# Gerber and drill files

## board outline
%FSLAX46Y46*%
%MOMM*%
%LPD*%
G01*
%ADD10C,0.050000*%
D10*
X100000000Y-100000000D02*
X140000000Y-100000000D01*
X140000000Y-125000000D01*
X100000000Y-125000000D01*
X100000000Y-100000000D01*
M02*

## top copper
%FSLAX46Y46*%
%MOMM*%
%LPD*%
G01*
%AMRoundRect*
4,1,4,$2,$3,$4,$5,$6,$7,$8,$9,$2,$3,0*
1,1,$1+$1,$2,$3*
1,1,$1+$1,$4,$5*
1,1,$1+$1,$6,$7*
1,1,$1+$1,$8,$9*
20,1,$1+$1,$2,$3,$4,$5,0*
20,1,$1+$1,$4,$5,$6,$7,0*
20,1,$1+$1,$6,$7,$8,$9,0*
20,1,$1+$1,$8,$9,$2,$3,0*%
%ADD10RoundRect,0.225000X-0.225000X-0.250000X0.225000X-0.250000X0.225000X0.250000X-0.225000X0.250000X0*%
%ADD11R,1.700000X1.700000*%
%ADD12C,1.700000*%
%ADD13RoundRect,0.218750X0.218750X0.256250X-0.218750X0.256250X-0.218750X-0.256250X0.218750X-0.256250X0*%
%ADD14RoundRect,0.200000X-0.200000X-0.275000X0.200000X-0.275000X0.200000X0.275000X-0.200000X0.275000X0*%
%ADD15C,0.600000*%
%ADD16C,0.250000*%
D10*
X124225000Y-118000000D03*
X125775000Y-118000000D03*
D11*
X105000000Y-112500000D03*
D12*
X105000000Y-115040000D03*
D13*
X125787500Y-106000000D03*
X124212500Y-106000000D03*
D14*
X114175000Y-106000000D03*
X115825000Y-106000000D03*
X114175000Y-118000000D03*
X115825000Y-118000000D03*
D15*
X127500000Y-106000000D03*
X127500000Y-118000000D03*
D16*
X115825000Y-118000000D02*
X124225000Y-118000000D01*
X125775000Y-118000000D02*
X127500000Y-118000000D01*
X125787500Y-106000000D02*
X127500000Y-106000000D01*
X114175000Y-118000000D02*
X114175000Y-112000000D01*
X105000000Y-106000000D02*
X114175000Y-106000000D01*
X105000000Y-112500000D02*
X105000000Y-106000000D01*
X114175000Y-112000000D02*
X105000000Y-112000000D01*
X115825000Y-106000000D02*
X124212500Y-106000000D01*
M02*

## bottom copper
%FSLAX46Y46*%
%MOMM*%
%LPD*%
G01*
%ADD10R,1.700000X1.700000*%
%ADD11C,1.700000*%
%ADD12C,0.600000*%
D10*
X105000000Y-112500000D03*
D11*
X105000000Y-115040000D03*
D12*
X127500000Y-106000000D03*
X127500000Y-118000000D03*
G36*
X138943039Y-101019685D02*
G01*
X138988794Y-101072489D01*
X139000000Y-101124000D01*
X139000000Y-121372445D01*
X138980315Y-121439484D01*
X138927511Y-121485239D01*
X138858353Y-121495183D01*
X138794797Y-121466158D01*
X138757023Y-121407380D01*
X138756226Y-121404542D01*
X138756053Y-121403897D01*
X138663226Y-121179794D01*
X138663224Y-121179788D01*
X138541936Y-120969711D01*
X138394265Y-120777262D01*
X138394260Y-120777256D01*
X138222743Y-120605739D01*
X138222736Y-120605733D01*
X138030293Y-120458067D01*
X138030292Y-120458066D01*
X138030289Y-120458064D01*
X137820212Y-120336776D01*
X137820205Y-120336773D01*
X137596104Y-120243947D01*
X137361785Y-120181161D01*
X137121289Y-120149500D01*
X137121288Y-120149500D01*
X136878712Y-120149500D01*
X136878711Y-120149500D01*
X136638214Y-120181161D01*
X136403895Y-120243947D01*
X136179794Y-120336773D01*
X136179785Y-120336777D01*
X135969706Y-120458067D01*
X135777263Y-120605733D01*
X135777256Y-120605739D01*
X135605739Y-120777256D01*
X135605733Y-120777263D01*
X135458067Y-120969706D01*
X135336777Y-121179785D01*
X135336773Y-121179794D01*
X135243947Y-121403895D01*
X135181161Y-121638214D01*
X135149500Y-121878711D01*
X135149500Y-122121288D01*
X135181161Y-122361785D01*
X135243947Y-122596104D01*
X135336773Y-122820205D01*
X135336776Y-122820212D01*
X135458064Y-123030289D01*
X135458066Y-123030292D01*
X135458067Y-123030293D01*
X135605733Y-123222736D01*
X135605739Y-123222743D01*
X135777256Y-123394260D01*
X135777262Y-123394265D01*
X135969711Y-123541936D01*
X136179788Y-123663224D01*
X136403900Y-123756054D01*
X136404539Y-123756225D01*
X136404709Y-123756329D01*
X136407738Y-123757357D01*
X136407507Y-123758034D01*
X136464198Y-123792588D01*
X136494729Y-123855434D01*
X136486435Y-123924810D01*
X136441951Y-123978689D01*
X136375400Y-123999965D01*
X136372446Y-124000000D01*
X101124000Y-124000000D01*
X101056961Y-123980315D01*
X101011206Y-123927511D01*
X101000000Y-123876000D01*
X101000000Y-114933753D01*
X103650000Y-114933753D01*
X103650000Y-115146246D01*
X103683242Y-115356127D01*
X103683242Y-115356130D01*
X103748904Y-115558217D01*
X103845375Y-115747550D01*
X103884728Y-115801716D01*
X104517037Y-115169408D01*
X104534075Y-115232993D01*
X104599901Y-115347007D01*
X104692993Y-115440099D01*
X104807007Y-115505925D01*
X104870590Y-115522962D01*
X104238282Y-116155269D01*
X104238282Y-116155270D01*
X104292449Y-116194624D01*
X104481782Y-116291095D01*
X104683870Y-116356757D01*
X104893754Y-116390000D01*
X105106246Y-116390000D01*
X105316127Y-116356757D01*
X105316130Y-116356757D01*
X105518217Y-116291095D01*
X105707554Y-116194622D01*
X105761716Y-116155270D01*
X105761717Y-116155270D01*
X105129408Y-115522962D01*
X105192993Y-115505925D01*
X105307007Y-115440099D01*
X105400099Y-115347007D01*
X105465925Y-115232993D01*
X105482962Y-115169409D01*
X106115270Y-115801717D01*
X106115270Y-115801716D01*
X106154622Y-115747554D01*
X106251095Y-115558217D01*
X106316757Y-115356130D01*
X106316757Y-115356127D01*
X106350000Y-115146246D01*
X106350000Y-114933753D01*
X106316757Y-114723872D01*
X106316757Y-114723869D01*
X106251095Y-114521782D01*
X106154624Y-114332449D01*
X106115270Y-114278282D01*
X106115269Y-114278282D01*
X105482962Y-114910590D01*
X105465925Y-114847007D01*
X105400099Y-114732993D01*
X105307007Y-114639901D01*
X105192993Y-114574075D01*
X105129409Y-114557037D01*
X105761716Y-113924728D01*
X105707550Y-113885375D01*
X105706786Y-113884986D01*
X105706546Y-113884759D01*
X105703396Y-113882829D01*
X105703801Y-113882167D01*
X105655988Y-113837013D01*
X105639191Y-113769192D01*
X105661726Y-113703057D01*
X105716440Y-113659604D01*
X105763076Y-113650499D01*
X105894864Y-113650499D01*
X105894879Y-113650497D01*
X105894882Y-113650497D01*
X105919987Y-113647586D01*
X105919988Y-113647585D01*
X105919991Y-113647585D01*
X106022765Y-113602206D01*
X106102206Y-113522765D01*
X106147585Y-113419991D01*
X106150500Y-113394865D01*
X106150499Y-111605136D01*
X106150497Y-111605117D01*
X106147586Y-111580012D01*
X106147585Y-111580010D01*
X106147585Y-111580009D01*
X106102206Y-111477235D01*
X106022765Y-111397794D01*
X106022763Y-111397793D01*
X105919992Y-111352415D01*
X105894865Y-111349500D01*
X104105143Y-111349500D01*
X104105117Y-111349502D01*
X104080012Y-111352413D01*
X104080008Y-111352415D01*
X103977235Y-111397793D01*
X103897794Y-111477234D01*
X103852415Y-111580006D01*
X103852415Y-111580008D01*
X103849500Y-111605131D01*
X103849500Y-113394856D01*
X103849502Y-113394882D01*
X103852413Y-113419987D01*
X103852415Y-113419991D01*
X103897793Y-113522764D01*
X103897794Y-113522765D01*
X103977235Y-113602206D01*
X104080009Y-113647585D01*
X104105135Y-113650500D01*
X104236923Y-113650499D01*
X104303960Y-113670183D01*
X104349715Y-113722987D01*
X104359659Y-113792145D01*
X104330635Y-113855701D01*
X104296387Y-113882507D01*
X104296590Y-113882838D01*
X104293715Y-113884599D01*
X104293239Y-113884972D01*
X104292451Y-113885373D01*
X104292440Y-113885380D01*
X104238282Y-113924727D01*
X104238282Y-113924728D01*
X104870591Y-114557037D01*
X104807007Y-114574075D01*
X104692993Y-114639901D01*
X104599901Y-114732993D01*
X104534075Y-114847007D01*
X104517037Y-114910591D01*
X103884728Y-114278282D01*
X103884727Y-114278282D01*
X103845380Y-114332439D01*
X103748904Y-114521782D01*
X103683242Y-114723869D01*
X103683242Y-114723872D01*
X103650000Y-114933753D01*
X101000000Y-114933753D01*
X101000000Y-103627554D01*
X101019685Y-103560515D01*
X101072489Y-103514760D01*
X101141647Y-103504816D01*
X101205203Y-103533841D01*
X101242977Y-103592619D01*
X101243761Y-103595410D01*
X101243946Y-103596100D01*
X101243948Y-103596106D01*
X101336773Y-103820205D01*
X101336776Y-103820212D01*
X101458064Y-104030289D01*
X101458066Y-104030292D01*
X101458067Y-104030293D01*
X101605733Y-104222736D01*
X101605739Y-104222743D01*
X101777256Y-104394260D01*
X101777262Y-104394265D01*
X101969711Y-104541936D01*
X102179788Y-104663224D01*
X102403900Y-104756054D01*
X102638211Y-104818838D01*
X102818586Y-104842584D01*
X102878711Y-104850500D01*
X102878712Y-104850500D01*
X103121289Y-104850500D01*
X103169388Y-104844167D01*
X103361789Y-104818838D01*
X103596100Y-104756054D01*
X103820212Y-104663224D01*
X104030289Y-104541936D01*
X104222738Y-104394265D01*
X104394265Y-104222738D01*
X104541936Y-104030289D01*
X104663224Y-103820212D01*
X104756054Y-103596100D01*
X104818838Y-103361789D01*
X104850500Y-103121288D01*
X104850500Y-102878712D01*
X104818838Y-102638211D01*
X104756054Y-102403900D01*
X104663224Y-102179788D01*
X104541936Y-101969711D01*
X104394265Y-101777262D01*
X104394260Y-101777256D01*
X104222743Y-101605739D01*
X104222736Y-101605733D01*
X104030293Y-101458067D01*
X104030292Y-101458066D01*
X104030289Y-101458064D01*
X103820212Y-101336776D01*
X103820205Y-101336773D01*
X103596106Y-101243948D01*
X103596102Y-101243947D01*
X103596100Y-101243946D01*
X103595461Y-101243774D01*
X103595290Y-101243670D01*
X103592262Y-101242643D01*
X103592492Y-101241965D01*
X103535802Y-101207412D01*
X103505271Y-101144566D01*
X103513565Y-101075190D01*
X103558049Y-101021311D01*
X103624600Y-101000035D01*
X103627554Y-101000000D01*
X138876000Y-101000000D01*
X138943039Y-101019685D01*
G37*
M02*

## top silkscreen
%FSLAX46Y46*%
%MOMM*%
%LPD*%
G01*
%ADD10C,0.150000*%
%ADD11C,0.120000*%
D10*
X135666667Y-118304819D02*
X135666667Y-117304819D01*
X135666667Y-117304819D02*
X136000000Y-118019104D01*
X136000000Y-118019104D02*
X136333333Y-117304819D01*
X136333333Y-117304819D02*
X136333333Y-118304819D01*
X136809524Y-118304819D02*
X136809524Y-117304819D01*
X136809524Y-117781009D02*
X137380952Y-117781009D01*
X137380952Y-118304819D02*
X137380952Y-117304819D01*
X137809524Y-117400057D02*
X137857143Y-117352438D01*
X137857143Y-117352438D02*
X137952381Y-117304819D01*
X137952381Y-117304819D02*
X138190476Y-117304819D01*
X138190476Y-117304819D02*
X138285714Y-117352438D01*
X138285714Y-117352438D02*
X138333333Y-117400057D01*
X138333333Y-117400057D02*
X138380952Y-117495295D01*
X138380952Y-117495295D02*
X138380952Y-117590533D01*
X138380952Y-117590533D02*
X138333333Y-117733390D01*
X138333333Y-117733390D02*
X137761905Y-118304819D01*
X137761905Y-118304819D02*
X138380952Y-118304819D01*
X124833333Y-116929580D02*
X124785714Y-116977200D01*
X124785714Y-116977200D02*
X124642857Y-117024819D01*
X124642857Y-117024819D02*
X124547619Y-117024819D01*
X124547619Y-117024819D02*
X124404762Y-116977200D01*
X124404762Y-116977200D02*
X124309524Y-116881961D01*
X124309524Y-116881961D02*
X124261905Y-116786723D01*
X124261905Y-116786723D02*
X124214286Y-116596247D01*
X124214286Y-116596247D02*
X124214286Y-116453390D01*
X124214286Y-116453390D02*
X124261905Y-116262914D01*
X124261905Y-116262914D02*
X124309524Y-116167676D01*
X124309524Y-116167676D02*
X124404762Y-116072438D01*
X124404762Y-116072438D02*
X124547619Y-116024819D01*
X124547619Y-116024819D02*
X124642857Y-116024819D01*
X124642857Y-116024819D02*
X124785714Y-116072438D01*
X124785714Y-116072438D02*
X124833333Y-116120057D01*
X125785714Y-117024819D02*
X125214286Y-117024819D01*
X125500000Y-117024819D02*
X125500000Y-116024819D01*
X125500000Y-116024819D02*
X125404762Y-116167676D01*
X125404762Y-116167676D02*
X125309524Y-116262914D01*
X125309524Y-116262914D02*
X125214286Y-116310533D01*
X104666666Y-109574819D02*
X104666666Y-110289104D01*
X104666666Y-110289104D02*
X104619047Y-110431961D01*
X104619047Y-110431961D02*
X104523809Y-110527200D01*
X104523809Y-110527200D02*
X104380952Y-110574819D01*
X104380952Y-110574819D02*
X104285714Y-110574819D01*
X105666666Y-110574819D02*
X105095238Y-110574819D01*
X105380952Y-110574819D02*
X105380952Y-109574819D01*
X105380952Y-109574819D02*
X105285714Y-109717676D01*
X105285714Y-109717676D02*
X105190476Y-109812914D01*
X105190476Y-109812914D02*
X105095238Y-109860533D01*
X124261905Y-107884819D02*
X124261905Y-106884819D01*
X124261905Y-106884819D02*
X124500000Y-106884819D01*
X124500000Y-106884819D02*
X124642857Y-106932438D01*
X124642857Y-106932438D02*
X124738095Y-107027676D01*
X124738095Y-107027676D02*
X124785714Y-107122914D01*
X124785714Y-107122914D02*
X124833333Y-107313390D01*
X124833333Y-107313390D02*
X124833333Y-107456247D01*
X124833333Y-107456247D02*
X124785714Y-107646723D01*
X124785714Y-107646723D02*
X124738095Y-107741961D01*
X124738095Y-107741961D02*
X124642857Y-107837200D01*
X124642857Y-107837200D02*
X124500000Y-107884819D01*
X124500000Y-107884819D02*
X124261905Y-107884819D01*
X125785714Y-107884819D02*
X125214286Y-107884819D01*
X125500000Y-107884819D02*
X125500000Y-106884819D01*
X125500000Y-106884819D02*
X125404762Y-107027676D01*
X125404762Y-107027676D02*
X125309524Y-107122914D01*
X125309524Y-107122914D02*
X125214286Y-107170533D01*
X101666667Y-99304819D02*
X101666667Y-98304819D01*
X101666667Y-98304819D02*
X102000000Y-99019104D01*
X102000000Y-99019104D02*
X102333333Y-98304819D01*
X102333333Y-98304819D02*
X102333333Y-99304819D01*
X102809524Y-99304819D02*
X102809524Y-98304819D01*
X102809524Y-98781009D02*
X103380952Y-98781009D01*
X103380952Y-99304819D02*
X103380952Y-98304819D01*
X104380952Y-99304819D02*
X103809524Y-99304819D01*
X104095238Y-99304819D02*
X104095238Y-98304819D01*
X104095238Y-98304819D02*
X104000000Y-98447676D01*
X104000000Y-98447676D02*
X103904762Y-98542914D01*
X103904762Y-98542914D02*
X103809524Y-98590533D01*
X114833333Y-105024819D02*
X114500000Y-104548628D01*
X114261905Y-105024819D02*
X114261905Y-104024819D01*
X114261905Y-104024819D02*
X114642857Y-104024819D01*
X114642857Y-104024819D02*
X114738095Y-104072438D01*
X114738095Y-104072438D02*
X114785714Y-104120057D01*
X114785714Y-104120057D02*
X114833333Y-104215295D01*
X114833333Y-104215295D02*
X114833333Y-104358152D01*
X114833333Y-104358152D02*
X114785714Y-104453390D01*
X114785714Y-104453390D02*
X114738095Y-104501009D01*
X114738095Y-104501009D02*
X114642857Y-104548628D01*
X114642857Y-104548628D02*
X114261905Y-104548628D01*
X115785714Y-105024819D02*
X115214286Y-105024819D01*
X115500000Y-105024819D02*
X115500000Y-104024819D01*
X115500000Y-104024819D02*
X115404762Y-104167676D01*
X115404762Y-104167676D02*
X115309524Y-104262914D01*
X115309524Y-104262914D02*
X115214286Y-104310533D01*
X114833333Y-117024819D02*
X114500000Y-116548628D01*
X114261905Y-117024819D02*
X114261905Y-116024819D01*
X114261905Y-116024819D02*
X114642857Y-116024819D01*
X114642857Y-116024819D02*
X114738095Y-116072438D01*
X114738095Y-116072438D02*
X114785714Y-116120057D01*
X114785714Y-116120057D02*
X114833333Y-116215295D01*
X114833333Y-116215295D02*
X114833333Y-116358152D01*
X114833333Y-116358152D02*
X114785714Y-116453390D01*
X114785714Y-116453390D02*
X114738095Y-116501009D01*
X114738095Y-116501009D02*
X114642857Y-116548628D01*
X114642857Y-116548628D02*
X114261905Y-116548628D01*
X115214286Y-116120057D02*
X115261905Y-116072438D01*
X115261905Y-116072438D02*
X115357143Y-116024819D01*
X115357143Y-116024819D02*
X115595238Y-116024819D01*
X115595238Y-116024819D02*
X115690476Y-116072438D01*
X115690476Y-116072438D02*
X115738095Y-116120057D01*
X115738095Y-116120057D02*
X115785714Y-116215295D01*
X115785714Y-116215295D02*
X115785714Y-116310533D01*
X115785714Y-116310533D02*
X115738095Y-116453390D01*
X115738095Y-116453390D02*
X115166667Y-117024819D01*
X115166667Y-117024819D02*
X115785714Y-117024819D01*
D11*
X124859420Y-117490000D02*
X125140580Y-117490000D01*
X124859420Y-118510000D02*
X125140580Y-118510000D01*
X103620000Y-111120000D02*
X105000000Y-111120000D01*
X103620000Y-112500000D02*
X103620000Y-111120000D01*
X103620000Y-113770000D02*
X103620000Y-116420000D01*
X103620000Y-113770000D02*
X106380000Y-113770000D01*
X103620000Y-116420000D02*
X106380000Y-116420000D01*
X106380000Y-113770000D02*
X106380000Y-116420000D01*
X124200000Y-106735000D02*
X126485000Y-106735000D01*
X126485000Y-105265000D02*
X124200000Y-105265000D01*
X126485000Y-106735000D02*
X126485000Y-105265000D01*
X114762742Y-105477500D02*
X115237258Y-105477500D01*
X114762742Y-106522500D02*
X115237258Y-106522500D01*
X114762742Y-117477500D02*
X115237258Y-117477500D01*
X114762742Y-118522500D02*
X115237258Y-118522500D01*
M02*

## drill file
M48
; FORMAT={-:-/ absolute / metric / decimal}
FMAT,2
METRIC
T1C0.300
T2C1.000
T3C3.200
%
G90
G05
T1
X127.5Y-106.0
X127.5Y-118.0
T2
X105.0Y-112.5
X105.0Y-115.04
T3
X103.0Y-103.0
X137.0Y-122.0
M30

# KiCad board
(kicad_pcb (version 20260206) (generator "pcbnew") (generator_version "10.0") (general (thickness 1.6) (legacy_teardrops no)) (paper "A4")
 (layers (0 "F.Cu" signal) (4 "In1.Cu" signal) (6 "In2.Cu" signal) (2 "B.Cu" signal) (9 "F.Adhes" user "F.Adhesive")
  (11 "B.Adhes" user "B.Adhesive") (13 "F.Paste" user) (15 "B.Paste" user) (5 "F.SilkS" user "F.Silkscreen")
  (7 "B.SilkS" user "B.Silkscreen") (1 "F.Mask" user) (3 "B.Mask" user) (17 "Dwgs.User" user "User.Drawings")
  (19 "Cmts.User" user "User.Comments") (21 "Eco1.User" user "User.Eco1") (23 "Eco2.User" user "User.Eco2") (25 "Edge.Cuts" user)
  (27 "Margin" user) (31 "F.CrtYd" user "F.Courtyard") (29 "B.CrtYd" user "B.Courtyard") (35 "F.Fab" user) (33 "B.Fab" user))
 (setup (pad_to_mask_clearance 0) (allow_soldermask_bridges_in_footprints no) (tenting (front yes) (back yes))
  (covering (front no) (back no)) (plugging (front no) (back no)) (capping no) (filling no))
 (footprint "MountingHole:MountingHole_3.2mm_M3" (layer "F.Cu") (at 137 122)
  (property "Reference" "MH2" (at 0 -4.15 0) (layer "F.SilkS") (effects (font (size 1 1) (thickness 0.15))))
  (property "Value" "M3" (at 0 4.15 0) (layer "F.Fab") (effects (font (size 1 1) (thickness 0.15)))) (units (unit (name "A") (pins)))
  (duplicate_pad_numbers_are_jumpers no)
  (pad "" np_thru_hole circle (at 0 0) (size 3.2 3.2) (drill 3.2) (layers "*.Cu" "*.Mask")))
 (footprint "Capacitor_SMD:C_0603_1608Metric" (layer "F.Cu") (at 125 118)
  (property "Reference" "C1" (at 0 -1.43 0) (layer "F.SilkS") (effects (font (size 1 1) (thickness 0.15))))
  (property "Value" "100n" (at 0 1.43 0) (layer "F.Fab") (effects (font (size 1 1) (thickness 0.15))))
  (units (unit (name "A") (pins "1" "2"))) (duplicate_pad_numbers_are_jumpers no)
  (fp_line (start -0.14058 -0.51) (end 0.14058 -0.51) (stroke (width 0.12) (type solid)) (layer "F.SilkS"))
  (fp_line (start -0.14058 0.51) (end 0.14058 0.51) (stroke (width 0.12) (type solid)) (layer "F.SilkS"))
  (pad "1" smd roundrect (at -0.775 0) (size 0.9 0.95) (layers "F.Cu" "F.Mask" "F.Paste") (roundrect_rratio 0.25) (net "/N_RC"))
  (pad "2" smd roundrect (at 0.775 0) (size 0.9 0.95) (layers "F.Cu" "F.Mask" "F.Paste") (roundrect_rratio 0.25) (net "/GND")))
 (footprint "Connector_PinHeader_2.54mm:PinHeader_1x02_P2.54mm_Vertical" (layer "F.Cu") (at 105 112.5)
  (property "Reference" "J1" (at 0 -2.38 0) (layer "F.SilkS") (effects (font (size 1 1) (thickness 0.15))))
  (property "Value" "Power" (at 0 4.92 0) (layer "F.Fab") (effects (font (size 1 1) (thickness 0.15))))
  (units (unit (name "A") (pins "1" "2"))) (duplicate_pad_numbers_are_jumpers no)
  (fp_line (start -1.38 -1.38) (end 0 -1.38) (stroke (width 0.12) (type solid)) (layer "F.SilkS"))
  (fp_line (start -1.38 0) (end -1.38 -1.38) (stroke (width 0.12) (type solid)) (layer "F.SilkS"))
  (fp_line (start -1.38 1.27) (end -1.38 3.92) (stroke (width 0.12) (type solid)) (layer "F.SilkS"))
  (fp_line (start -1.38 1.27) (end 1.38 1.27) (stroke (width 0.12) (type solid)) (layer "F.SilkS"))
  (fp_line (start -1.38 3.92) (end 1.38 3.92) (stroke (width 0.12) (type solid)) (layer "F.SilkS"))
  (fp_line (start 1.38 1.27) (end 1.38 3.92) (stroke (width 0.12) (type solid)) (layer "F.SilkS"))
  (pad "1" thru_hole rect (at 0 0) (size 1.7 1.7) (drill 1) (layers "*.Cu" "*.Mask") (remove_unused_layers no) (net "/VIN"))
  (pad "2" thru_hole circle (at 0 2.54) (size 1.7 1.7) (drill 1) (layers "*.Cu" "*.Mask") (remove_unused_layers no) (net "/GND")))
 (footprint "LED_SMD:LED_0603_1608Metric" (layer "F.Cu") (at 125 106 180)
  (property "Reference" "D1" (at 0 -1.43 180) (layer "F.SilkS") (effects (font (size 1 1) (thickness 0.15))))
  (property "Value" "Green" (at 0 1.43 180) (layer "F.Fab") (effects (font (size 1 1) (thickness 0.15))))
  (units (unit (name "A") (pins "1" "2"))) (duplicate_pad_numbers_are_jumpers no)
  (fp_line (start 0.8 -0.735) (end -1.485 -0.735) (stroke (width 0.12) (type solid)) (layer "F.SilkS"))
  (fp_line (start -1.485 0.735) (end 0.8 0.735) (stroke (width 0.12) (type solid)) (layer "F.SilkS"))
  (fp_line (start -1.485 -0.735) (end -1.485 0.735) (stroke (width 0.12) (type solid)) (layer "F.SilkS"))
  (pad "1" smd roundrect (at -0.7875 0 180) (size 0.875 0.95) (layers "F.Cu" "F.Mask" "F.Paste") (roundrect_rratio 0.25) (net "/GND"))
  (pad "2" smd roundrect (at 0.7875 0 180) (size 0.875 0.95) (layers "F.Cu" "F.Mask" "F.Paste") (roundrect_rratio 0.25) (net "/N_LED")))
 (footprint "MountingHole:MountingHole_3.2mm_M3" (layer "F.Cu") (at 103 103)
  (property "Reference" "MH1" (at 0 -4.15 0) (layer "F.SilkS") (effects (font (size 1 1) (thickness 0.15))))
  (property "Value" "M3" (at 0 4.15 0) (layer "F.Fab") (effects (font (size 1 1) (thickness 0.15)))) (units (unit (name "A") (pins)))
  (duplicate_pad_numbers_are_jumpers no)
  (pad "" np_thru_hole circle (at 0 0) (size 3.2 3.2) (drill 3.2) (layers "*.Cu" "*.Mask")))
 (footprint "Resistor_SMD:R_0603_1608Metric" (layer "F.Cu") (at 115 106)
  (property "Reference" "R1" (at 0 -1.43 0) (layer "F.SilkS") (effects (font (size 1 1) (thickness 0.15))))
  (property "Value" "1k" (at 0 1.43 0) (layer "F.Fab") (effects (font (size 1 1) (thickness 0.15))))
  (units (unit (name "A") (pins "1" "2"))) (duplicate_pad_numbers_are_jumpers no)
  (fp_line (start -0.237258 -0.5225) (end 0.237258 -0.5225) (stroke (width 0.12) (type solid)) (layer "F.SilkS"))
  (fp_line (start -0.237258 0.5225) (end 0.237258 0.5225) (stroke (width 0.12) (type solid)) (layer "F.SilkS"))
  (pad "1" smd roundrect (at -0.825 0) (size 0.8 0.95) (layers "F.Cu" "F.Mask" "F.Paste") (roundrect_rratio 0.25) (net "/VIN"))
  (pad "2" smd roundrect (at 0.825 0) (size 0.8 0.95) (layers "F.Cu" "F.Mask" "F.Paste") (roundrect_rratio 0.25) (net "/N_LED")))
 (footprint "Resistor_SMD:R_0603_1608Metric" (layer "F.Cu") (at 115 118)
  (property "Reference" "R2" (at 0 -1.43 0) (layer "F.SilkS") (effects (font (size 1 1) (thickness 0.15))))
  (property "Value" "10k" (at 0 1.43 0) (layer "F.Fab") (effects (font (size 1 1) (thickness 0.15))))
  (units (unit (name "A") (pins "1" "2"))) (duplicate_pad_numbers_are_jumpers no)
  (fp_line (start -0.237258 -0.5225) (end 0.237258 -0.5225) (stroke (width 0.12) (type solid)) (layer "F.SilkS"))
  (fp_line (start -0.237258 0.5225) (end 0.237258 0.5225) (stroke (width 0.12) (type solid)) (layer "F.SilkS"))
  (pad "1" smd roundrect (at -0.825 0) (size 0.8 0.95) (layers "F.Cu" "F.Mask" "F.Paste") (roundrect_rratio 0.25) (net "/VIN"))
  (pad "2" smd roundrect (at 0.825 0) (size 0.8 0.95) (layers "F.Cu" "F.Mask" "F.Paste") (roundrect_rratio 0.25) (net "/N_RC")))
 (gr_rect (start 100 100) (end 140 125) (stroke (width 0.05) (type default)) (fill no) (layer "Edge.Cuts"))
 (segment (start 115.825 118) (end 124.225 118) (width 0.25) (layer "F.Cu") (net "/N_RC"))
 (segment (start 125.775 118) (end 127.5 118) (width 0.25) (layer "F.Cu") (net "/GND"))
 (segment (start 125.7875 106) (end 127.5 106) (width 0.25) (layer "F.Cu") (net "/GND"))
 (via (at 127.5 106) (size 0.6) (drill 0.3) (layers "F.Cu" "B.Cu") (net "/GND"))
 (via (at 127.5 118) (size 0.6) (drill 0.3) (layers "F.Cu" "B.Cu") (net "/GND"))
 (segment (start 114.175 118) (end 114.175 112) (width 0.25) (layer "F.Cu") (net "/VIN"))
 (segment (start 105 106) (end 114.175 106) (width 0.25) (layer "F.Cu") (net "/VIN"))
 (segment (start 105 112.5) (end 105 106) (width 0.25) (layer "F.Cu") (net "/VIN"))
 (segment (start 114.175 112) (end 105 112) (width 0.25) (layer "F.Cu") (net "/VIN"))
 (segment (start 115.825 106) (end 124.2125 106) (width 0.25) (layer "F.Cu") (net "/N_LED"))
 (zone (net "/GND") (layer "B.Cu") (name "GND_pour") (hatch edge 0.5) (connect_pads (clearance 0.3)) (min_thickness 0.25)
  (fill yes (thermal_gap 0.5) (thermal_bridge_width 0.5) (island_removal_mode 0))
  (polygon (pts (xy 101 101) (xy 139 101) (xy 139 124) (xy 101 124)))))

